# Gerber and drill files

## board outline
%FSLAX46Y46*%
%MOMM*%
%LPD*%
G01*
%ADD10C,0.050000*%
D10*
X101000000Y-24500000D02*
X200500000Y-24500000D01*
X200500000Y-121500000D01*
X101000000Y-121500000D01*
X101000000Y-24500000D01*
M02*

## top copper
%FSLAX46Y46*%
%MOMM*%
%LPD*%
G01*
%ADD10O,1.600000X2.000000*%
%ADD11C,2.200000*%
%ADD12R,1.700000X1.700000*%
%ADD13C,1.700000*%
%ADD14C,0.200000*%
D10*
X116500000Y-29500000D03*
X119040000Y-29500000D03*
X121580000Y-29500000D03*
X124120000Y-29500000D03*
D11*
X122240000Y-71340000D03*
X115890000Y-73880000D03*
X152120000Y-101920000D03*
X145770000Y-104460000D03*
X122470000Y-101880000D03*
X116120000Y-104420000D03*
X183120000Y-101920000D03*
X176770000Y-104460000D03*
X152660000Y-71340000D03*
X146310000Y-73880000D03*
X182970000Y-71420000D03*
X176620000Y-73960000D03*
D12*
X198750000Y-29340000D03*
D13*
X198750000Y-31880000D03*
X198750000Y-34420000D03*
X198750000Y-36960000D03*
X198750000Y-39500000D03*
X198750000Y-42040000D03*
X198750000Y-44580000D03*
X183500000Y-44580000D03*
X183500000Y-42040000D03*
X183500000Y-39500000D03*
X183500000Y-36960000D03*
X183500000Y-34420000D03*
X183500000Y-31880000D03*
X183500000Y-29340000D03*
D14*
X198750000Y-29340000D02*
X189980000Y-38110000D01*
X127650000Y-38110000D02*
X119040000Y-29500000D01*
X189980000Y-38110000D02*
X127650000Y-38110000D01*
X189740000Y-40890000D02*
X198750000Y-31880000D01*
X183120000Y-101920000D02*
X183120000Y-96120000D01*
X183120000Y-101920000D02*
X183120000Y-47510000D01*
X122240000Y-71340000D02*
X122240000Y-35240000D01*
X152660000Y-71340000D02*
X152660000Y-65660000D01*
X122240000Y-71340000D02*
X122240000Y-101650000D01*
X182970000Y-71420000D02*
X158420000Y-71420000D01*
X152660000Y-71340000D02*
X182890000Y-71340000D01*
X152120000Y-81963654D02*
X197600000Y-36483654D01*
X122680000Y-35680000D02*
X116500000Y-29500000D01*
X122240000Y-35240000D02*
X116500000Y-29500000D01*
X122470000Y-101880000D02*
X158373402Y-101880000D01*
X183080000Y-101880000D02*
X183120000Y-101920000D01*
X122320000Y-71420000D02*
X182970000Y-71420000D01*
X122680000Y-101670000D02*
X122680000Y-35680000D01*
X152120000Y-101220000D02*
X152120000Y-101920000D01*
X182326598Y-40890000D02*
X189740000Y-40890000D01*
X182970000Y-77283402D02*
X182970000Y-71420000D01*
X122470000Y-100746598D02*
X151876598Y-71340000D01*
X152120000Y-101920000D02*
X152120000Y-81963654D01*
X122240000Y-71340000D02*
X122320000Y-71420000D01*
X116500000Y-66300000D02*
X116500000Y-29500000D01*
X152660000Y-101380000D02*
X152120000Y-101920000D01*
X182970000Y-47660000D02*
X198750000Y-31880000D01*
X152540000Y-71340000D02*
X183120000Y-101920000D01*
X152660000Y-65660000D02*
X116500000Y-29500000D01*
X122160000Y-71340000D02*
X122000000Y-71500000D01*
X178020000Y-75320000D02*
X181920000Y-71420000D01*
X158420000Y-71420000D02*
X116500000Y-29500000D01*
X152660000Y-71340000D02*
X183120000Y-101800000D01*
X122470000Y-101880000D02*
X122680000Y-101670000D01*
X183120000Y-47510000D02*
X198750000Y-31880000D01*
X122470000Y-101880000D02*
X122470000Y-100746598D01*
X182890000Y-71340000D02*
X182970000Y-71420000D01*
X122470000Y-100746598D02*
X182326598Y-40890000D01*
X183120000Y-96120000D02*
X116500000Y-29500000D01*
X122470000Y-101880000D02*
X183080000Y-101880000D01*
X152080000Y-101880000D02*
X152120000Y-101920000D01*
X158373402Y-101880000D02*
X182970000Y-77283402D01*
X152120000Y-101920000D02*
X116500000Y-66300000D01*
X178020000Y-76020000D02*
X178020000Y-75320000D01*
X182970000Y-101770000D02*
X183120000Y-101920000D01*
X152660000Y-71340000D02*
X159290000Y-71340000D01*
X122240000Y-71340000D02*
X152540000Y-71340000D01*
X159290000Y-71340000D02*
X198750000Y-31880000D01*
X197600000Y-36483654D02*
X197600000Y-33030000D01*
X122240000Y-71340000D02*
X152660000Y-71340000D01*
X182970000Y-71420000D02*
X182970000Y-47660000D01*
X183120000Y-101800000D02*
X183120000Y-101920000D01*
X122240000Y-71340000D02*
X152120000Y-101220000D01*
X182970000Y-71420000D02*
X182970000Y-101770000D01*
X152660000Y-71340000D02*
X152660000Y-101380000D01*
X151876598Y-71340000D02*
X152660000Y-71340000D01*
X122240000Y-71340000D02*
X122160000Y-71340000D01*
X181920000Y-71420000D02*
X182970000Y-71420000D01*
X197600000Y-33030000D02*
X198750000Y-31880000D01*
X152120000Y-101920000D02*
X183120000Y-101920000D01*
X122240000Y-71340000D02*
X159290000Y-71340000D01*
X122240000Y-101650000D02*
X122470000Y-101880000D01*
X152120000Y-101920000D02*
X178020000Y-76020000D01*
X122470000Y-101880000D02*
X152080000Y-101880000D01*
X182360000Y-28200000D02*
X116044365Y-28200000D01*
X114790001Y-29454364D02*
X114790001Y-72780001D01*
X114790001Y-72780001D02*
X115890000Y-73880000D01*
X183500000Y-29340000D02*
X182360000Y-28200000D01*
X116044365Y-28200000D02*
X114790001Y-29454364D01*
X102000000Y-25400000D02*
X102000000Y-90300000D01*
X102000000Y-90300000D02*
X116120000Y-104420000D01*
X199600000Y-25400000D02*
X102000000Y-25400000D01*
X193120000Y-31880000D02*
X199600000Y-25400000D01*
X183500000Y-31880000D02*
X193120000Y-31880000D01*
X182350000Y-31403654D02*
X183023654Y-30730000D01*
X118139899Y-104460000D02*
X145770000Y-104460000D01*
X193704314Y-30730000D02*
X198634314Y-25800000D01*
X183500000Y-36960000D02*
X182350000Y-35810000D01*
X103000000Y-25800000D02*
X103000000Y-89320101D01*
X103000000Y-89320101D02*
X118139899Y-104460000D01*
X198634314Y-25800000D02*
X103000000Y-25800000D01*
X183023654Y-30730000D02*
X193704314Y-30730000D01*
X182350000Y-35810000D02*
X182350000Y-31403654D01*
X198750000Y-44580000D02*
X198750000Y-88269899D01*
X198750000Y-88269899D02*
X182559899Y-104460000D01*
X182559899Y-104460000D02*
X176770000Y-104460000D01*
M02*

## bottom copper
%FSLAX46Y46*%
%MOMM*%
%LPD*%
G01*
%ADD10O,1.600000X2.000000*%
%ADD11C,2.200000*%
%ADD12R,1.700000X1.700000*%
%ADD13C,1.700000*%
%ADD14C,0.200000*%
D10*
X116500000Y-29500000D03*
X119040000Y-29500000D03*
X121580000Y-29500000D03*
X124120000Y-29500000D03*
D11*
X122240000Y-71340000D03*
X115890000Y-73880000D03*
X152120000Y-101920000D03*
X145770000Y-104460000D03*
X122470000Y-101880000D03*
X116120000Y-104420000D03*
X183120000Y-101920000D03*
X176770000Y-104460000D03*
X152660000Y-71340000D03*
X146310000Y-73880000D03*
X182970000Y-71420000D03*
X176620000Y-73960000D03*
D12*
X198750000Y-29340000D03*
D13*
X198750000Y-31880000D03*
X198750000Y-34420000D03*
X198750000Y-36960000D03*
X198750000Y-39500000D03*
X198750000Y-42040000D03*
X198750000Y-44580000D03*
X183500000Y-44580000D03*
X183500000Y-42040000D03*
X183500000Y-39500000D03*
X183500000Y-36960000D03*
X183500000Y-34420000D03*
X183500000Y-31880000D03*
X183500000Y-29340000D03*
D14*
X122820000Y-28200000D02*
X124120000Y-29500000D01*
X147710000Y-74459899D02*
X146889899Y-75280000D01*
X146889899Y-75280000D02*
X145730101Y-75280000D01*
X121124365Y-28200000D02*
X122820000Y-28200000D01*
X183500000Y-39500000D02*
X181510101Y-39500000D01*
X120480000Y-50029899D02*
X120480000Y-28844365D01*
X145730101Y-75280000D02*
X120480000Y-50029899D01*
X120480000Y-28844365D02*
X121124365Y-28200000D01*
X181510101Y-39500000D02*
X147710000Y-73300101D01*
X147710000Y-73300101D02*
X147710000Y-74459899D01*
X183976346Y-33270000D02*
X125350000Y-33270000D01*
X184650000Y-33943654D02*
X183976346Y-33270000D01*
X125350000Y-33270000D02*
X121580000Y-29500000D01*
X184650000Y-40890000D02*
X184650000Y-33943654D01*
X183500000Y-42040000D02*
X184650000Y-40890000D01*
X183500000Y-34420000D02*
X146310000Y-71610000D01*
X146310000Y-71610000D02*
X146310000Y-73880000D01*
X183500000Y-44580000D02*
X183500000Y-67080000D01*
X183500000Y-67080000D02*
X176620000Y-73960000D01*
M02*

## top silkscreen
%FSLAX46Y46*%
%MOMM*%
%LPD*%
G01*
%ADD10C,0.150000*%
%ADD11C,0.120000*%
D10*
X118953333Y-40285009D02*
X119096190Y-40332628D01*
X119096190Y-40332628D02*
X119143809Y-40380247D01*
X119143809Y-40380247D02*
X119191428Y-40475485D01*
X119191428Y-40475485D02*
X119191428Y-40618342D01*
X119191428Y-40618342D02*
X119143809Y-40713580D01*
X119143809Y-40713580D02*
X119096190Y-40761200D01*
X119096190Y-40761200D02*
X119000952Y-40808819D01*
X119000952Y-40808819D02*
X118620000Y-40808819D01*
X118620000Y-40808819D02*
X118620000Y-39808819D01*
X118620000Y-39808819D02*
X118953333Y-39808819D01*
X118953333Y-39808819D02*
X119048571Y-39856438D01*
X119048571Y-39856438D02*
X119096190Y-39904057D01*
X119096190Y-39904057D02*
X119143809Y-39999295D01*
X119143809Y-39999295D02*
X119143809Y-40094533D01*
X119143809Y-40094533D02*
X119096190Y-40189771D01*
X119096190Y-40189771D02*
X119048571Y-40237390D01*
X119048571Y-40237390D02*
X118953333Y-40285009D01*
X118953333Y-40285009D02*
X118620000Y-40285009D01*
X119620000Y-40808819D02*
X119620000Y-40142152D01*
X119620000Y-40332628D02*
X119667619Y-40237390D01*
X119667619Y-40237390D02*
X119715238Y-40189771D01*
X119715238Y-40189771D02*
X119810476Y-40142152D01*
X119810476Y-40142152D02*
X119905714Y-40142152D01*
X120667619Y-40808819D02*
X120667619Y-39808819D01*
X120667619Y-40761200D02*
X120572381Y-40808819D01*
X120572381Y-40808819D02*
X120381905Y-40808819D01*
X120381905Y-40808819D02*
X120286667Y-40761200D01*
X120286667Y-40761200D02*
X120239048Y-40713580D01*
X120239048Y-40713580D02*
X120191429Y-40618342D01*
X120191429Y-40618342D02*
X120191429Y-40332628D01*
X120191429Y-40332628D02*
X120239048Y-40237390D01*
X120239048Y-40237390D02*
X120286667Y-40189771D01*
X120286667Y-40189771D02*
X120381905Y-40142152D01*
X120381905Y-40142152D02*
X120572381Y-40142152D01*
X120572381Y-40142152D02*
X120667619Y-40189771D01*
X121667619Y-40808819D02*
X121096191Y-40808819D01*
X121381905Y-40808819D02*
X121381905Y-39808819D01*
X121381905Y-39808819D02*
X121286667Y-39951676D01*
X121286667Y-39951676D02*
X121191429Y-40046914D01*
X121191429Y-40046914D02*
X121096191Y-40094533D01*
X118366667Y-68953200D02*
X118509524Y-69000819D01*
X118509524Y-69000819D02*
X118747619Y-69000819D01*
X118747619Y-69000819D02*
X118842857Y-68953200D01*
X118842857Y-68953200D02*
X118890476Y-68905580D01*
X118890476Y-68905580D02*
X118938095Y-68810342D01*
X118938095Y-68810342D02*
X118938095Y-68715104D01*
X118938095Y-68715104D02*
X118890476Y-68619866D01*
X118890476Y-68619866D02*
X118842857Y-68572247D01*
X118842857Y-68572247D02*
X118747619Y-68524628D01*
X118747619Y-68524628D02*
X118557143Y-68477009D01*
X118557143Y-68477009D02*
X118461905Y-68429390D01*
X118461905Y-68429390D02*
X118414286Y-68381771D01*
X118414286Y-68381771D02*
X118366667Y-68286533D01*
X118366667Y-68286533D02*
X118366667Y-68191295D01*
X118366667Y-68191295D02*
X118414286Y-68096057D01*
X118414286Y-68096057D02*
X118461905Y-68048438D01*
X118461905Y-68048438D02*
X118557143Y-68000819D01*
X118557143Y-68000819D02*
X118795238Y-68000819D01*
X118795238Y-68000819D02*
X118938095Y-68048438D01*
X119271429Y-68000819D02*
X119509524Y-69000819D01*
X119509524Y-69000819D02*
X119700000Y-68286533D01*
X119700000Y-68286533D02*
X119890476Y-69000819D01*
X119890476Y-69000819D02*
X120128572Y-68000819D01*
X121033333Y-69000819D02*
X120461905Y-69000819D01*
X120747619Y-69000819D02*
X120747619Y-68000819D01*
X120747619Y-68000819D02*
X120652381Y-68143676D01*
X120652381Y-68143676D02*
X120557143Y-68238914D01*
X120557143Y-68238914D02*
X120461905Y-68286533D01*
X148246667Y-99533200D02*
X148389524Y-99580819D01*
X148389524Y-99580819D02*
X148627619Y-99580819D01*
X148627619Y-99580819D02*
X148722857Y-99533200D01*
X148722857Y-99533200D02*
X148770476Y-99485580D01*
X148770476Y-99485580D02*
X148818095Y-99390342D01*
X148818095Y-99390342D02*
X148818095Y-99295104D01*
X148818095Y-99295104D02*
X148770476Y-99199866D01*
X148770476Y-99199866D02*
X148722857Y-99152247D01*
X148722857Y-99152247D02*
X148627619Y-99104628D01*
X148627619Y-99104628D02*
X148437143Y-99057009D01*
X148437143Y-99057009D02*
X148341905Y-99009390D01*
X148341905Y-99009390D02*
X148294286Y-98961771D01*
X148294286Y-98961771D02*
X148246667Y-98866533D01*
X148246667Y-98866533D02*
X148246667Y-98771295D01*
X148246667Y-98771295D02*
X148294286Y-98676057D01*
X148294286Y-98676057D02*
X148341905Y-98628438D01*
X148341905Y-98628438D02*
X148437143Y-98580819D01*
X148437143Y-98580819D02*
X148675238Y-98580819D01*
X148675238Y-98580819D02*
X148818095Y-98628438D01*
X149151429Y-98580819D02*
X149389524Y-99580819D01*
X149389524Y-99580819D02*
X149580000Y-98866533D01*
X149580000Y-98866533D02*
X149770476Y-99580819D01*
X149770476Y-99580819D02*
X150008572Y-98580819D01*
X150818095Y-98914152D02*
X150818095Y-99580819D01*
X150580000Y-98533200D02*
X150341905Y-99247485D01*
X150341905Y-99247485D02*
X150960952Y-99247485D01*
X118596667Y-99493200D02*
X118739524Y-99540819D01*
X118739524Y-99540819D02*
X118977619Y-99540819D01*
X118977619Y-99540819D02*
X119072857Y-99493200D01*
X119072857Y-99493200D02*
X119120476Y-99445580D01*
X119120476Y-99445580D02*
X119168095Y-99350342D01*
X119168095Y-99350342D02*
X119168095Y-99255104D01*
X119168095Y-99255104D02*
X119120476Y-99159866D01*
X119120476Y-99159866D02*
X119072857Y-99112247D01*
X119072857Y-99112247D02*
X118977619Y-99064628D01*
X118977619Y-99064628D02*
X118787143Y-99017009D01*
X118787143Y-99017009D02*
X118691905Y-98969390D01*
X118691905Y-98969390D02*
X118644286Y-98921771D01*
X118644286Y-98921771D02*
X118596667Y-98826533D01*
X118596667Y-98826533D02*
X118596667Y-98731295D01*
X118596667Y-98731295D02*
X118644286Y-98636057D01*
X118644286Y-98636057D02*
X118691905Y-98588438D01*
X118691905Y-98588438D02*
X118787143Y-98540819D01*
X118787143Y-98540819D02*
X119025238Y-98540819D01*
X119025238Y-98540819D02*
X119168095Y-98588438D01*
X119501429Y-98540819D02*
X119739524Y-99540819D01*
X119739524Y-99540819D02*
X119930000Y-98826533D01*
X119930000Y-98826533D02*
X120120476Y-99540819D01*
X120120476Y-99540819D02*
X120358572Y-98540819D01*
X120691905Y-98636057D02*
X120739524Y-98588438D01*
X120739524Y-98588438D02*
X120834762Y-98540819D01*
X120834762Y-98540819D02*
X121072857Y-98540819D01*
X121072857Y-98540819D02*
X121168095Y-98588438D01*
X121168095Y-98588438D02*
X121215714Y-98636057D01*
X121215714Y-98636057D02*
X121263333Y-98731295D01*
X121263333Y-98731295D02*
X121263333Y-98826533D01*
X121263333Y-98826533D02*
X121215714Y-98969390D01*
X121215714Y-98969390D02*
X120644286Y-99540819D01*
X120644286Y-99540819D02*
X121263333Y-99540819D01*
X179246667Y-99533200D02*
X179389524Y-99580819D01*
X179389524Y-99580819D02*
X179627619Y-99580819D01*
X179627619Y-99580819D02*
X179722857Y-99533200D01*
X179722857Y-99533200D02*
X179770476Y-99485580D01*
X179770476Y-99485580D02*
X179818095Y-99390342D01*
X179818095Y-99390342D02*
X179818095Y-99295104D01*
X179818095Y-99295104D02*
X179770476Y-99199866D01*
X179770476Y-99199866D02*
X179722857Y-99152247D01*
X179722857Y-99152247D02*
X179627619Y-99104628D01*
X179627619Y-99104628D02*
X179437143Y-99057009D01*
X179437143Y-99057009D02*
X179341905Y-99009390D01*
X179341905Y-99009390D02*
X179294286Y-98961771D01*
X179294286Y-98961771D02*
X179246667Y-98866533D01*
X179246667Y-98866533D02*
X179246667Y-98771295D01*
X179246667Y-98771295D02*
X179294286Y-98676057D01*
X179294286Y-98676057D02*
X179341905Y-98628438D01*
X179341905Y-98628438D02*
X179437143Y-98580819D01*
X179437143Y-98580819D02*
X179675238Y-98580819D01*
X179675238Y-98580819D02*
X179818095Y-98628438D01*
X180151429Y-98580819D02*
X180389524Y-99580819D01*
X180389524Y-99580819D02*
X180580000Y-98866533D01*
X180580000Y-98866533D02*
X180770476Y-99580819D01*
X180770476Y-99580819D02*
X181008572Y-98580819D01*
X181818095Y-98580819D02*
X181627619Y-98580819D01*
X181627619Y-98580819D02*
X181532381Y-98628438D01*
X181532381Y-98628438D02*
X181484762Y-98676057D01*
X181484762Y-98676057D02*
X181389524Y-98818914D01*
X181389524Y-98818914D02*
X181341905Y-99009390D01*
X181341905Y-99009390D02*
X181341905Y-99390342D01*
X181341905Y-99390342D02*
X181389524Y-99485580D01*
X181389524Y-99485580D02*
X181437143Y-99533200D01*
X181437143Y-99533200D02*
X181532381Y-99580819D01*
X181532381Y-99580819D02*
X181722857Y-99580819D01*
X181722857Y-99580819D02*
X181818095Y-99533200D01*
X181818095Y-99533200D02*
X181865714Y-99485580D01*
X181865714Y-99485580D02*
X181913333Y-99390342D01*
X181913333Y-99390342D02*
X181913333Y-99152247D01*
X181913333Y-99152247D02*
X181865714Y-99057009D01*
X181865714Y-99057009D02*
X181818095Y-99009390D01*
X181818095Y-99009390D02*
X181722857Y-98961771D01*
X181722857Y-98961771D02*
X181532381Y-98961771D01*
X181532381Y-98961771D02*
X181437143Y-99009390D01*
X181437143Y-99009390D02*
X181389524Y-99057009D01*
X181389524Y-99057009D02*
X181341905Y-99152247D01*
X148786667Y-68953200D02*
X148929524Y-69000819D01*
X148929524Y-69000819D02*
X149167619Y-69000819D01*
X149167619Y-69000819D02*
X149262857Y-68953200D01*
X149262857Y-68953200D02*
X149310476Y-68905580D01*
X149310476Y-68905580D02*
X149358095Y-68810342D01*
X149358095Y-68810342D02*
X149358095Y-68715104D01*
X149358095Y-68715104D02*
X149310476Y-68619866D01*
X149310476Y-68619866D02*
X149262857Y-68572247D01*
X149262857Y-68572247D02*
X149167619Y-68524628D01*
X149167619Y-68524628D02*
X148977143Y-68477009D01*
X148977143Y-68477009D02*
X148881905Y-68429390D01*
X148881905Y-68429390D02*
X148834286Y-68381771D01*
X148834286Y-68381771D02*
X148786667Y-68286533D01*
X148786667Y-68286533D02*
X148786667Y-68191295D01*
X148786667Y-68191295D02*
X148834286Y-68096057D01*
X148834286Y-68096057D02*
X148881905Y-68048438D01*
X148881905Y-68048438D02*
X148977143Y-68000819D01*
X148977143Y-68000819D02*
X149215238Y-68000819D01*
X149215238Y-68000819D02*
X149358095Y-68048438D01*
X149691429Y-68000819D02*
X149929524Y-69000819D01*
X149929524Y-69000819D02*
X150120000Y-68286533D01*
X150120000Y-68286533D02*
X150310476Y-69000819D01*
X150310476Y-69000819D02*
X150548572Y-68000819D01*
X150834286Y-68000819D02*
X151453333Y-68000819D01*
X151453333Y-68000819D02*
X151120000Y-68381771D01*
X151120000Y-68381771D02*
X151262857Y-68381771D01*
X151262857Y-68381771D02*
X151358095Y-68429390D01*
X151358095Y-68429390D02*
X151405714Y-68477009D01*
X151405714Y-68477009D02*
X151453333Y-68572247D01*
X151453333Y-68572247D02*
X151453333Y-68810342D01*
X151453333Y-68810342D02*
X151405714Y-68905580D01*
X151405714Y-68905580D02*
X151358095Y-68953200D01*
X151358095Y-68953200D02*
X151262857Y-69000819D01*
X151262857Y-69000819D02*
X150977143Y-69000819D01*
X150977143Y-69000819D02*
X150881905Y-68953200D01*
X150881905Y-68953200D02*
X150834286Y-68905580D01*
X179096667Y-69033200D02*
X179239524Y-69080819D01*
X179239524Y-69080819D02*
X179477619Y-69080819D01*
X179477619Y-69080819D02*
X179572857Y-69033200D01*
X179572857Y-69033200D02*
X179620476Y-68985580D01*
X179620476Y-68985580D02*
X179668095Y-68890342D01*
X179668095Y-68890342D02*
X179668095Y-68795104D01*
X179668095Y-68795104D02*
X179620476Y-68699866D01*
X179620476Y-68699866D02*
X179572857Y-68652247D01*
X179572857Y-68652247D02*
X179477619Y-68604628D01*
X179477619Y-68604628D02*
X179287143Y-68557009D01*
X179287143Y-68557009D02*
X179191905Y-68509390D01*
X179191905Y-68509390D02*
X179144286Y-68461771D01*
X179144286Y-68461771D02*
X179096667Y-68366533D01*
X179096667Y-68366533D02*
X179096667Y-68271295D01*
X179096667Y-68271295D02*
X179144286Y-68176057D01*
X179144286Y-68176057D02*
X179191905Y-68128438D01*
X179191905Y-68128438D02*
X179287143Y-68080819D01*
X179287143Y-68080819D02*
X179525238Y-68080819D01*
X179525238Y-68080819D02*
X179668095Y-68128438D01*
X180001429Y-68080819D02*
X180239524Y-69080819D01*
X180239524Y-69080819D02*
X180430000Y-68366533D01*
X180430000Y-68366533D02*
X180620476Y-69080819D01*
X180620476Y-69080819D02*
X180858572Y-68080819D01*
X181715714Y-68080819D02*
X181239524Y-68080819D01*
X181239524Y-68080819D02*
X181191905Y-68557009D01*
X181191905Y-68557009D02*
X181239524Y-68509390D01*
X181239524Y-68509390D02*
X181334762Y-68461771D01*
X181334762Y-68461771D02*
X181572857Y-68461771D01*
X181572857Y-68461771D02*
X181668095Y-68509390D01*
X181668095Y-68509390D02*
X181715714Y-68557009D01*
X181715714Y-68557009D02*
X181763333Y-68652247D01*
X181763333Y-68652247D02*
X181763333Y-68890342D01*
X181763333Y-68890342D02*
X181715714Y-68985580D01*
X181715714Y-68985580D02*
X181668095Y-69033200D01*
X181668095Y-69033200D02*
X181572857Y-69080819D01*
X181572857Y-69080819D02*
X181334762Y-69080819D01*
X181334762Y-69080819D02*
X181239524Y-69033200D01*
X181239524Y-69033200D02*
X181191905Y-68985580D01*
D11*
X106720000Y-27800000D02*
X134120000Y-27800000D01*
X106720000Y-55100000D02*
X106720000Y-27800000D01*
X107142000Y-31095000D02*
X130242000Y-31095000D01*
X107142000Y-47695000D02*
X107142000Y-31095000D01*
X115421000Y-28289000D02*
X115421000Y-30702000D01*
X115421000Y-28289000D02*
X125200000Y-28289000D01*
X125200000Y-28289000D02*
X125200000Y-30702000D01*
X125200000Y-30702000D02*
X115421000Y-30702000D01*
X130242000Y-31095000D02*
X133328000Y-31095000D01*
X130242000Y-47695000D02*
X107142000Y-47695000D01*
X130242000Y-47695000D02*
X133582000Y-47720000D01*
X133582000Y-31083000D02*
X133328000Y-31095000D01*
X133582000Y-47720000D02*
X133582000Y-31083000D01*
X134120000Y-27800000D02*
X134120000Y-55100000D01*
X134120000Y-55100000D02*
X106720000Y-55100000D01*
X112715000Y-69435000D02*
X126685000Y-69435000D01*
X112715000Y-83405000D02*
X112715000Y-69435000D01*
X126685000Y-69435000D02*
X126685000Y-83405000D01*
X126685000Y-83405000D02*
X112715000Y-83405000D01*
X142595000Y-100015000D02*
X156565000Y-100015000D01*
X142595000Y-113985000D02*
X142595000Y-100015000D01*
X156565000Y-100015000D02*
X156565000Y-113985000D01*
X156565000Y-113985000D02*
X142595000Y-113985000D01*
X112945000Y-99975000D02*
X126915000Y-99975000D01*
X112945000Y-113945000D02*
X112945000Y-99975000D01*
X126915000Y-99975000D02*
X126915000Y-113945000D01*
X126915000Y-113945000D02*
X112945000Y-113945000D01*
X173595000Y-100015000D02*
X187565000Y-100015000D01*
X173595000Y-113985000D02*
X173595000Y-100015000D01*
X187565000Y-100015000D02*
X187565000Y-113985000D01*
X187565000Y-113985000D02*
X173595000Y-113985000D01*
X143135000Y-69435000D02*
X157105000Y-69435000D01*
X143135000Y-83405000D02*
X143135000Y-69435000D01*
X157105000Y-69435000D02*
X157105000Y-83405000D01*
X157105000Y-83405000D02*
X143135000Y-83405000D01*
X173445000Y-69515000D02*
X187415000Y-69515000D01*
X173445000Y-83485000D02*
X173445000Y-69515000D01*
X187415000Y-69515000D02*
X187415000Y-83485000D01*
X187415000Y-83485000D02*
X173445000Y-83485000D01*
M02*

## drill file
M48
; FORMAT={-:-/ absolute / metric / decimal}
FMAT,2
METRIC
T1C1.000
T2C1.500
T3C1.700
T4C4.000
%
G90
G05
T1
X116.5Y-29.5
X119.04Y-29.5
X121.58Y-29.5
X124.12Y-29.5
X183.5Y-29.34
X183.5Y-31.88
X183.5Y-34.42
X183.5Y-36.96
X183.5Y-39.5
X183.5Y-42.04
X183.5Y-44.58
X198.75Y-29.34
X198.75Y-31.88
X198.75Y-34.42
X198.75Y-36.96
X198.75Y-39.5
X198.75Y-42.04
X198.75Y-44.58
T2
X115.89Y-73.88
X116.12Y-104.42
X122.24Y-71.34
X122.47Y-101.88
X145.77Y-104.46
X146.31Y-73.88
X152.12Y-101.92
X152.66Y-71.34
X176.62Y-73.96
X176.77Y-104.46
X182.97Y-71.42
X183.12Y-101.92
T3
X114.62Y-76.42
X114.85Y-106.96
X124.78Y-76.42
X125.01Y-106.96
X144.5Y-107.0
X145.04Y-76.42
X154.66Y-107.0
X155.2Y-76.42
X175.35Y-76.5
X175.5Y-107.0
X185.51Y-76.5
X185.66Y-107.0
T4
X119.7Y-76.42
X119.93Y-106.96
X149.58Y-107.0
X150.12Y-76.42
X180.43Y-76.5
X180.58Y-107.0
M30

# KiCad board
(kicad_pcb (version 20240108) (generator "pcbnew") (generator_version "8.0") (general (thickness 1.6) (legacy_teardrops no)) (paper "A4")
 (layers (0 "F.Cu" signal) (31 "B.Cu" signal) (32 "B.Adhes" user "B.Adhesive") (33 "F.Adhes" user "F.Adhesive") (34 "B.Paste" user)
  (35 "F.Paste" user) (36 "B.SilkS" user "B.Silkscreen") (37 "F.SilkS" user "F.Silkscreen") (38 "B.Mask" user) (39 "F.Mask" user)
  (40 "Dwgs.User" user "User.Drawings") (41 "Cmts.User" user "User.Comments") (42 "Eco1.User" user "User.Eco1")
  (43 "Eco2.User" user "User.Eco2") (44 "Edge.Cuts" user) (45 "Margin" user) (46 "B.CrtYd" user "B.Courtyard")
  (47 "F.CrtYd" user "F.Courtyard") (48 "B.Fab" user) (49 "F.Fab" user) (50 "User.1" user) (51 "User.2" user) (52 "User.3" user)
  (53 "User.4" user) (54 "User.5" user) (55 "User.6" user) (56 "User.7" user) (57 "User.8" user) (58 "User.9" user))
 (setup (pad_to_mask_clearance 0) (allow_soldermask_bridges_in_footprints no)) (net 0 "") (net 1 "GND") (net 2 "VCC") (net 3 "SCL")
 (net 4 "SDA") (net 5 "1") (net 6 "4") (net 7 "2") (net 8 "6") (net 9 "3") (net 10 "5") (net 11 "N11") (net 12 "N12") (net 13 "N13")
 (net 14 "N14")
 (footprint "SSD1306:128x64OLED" (layer "F.Cu") (at 120.12 40.1)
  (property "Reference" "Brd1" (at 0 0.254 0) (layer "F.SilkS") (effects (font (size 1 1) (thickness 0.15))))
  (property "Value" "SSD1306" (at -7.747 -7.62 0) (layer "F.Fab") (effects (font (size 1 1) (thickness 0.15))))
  (fp_line (start -13.4 -12.3) (end 14 -12.3) (stroke (width 0.12) (type solid)) (layer "F.SilkS"))
  (fp_line (start -13.4 15) (end -13.4 -12.3) (stroke (width 0.12) (type solid)) (layer "F.SilkS"))
  (fp_line (start -12.978 -9.005) (end 10.122 -9.005) (stroke (width 0.12) (type solid)) (layer "F.SilkS"))
  (fp_line (start -12.978 7.595) (end -12.978 -9.005) (stroke (width 0.12) (type solid)) (layer "F.SilkS"))
  (fp_line (start -4.699 -11.811) (end -4.699 -9.398) (stroke (width 0.12) (type solid)) (layer "F.SilkS"))
  (fp_line (start -4.699 -11.811) (end 5.08 -11.811) (stroke (width 0.12) (type solid)) (layer "F.SilkS"))
  (fp_line (start 5.08 -11.811) (end 5.08 -9.398) (stroke (width 0.12) (type solid)) (layer "F.SilkS"))
  (fp_line (start 5.08 -9.398) (end -4.699 -9.398) (stroke (width 0.12) (type solid)) (layer "F.SilkS"))
  (fp_line (start 10.122 -9.005) (end 13.208 -9.005) (stroke (width 0.12) (type solid)) (layer "F.SilkS"))
  (fp_line (start 10.122 7.595) (end -12.978 7.595) (stroke (width 0.12) (type solid)) (layer "F.SilkS"))
  (fp_line (start 10.122 7.595) (end 13.462 7.62) (stroke (width 0.12) (type solid)) (layer "F.SilkS"))
  (fp_line (start 13.462 -9.017) (end 13.208 -9.005) (stroke (width 0.12) (type solid)) (layer "F.SilkS"))
  (fp_line (start 13.462 7.62) (end 13.462 -9.017) (stroke (width 0.12) (type solid)) (layer "F.SilkS"))
  (fp_line (start 14 -12.3) (end 14 15) (stroke (width 0.12) (type solid)) (layer "F.SilkS"))
  (fp_line (start 14 15) (end -13.4 15) (stroke (width 0.12) (type solid)) (layer "F.SilkS"))
  (pad "1" thru_hole oval (at -3.62 -10.6 90) (size 2 1.6) (drill 1) (layers "*.Cu" "*.Mask") (remove_unused_layers no) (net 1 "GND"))
  (pad "2" thru_hole oval (at -1.08 -10.6 90) (size 2 1.6) (drill 1) (layers "*.Cu" "*.Mask") (remove_unused_layers no) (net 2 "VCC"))
  (pad "3" thru_hole oval (at 1.46 -10.6 90) (size 2 1.6) (drill 1) (layers "*.Cu" "*.Mask") (remove_unused_layers no) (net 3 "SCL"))
  (pad "4" thru_hole oval (at 4 -10.6 90) (size 2 1.6) (drill 1) (layers "*.Cu" "*.Mask") (remove_unused_layers no) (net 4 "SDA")))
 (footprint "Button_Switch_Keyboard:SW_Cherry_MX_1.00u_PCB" (layer "F.Cu") (at 122.24 71.34)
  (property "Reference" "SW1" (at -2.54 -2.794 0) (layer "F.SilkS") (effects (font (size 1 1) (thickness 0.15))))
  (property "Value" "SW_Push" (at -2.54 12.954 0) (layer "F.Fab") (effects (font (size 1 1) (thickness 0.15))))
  (fp_line (start -9.525 -1.905) (end 4.445 -1.905) (stroke (width 0.12) (type solid)) (layer "F.SilkS"))
  (fp_line (start -9.525 12.065) (end -9.525 -1.905) (stroke (width 0.12) (type solid)) (layer "F.SilkS"))
  (fp_line (start 4.445 -1.905) (end 4.445 12.065) (stroke (width 0.12) (type solid)) (layer "F.SilkS"))
  (fp_line (start 4.445 12.065) (end -9.525 12.065) (stroke (width 0.12) (type solid)) (layer "F.SilkS"))
  (pad "" np_thru_hole circle (at -7.62 5.08) (size 1.7 1.7) (drill 1.7) (layers "*.Cu" "*.Mask"))
  (pad "" np_thru_hole circle (at -2.54 5.08) (size 4 4) (drill 4) (layers "*.Cu" "*.Mask"))
  (pad "" np_thru_hole circle (at 2.54 5.08) (size 1.7 1.7) (drill 1.7) (layers "*.Cu" "*.Mask"))
  (pad "1" thru_hole circle (at 0 0) (size 2.2 2.2) (drill 1.5) (layers "*.Cu" "*.Mask") (remove_unused_layers no) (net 1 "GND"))
  (pad "2" thru_hole circle (at -6.35 2.54) (size 2.2 2.2) (drill 1.5) (layers "*.Cu" "*.Mask") (remove_unused_layers no) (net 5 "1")))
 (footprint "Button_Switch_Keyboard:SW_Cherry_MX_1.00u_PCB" (layer "F.Cu") (at 152.12 101.92)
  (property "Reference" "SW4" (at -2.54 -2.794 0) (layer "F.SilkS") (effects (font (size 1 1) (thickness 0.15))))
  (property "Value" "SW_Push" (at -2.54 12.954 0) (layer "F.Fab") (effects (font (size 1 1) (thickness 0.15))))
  (fp_line (start -9.525 -1.905) (end 4.445 -1.905) (stroke (width 0.12) (type solid)) (layer "F.SilkS"))
  (fp_line (start -9.525 12.065) (end -9.525 -1.905) (stroke (width 0.12) (type solid)) (layer "F.SilkS"))
  (fp_line (start 4.445 -1.905) (end 4.445 12.065) (stroke (width 0.12) (type solid)) (layer "F.SilkS"))
  (fp_line (start 4.445 12.065) (end -9.525 12.065) (stroke (width 0.12) (type solid)) (layer "F.SilkS"))
  (pad "" np_thru_hole circle (at -7.62 5.08) (size 1.7 1.7) (drill 1.7) (layers "*.Cu" "*.Mask"))
  (pad "" np_thru_hole circle (at -2.54 5.08) (size 4 4) (drill 4) (layers "*.Cu" "*.Mask"))
  (pad "" np_thru_hole circle (at 2.54 5.08) (size 1.7 1.7) (drill 1.7) (layers "*.Cu" "*.Mask"))
  (pad "1" thru_hole circle (at 0 0) (size 2.2 2.2) (drill 1.5) (layers "*.Cu" "*.Mask") (remove_unused_layers no) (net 1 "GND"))
  (pad "2" thru_hole circle (at -6.35 2.54) (size 2.2 2.2) (drill 1.5) (layers "*.Cu" "*.Mask") (remove_unused_layers no) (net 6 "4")))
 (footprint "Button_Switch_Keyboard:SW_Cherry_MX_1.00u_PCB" (layer "F.Cu") (at 122.47 101.88)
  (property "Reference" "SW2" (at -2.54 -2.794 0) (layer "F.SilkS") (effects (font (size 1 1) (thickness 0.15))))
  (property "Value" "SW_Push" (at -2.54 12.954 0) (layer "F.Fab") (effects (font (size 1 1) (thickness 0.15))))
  (fp_line (start -9.525 -1.905) (end 4.445 -1.905) (stroke (width 0.12) (type solid)) (layer "F.SilkS"))
  (fp_line (start -9.525 12.065) (end -9.525 -1.905) (stroke (width 0.12) (type solid)) (layer "F.SilkS"))
  (fp_line (start 4.445 -1.905) (end 4.445 12.065) (stroke (width 0.12) (type solid)) (layer "F.SilkS"))
  (fp_line (start 4.445 12.065) (end -9.525 12.065) (stroke (width 0.12) (type solid)) (layer "F.SilkS"))
  (pad "" np_thru_hole circle (at -7.62 5.08) (size 1.7 1.7) (drill 1.7) (layers "*.Cu" "*.Mask"))
  (pad "" np_thru_hole circle (at -2.54 5.08) (size 4 4) (drill 4) (layers "*.Cu" "*.Mask"))
  (pad "" np_thru_hole circle (at 2.54 5.08) (size 1.7 1.7) (drill 1.7) (layers "*.Cu" "*.Mask"))
  (pad "1" thru_hole circle (at 0 0) (size 2.2 2.2) (drill 1.5) (layers "*.Cu" "*.Mask") (remove_unused_layers no) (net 1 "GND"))
  (pad "2" thru_hole circle (at -6.35 2.54) (size 2.2 2.2) (drill 1.5) (layers "*.Cu" "*.Mask") (remove_unused_layers no) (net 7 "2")))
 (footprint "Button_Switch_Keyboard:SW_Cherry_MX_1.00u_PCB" (layer "F.Cu") (at 183.12 101.92)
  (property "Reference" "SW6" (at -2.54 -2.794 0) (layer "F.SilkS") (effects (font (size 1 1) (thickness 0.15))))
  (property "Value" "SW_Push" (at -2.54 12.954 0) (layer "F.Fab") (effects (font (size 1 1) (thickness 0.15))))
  (fp_line (start -9.525 -1.905) (end 4.445 -1.905) (stroke (width 0.12) (type solid)) (layer "F.SilkS"))
  (fp_line (start -9.525 12.065) (end -9.525 -1.905) (stroke (width 0.12) (type solid)) (layer "F.SilkS"))
  (fp_line (start 4.445 -1.905) (end 4.445 12.065) (stroke (width 0.12) (type solid)) (layer "F.SilkS"))
  (fp_line (start 4.445 12.065) (end -9.525 12.065) (stroke (width 0.12) (type solid)) (layer "F.SilkS"))
  (pad "" np_thru_hole circle (at -7.62 5.08) (size 1.7 1.7) (drill 1.7) (layers "*.Cu" "*.Mask"))
  (pad "" np_thru_hole circle (at -2.54 5.08) (size 4 4) (drill 4) (layers "*.Cu" "*.Mask"))
  (pad "" np_thru_hole circle (at 2.54 5.08) (size 1.7 1.7) (drill 1.7) (layers "*.Cu" "*.Mask"))
  (pad "1" thru_hole circle (at 0 0) (size 2.2 2.2) (drill 1.5) (layers "*.Cu" "*.Mask") (remove_unused_layers no) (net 1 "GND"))
  (pad "2" thru_hole circle (at -6.35 2.54) (size 2.2 2.2) (drill 1.5) (layers "*.Cu" "*.Mask") (remove_unused_layers no) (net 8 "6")))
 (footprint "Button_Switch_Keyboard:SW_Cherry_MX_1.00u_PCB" (layer "F.Cu") (at 152.66 71.34)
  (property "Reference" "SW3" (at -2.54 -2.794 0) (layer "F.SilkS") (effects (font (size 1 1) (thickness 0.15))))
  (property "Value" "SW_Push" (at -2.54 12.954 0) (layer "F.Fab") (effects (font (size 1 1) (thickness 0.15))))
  (fp_line (start -9.525 -1.905) (end 4.445 -1.905) (stroke (width 0.12) (type solid)) (layer "F.SilkS"))
  (fp_line (start -9.525 12.065) (end -9.525 -1.905) (stroke (width 0.12) (type solid)) (layer "F.SilkS"))
  (fp_line (start 4.445 -1.905) (end 4.445 12.065) (stroke (width 0.12) (type solid)) (layer "F.SilkS"))
  (fp_line (start 4.445 12.065) (end -9.525 12.065) (stroke (width 0.12) (type solid)) (layer "F.SilkS"))
  (pad "" np_thru_hole circle (at -7.62 5.08) (size 1.7 1.7) (drill 1.7) (layers "*.Cu" "*.Mask"))
  (pad "" np_thru_hole circle (at -2.54 5.08) (size 4 4) (drill 4) (layers "*.Cu" "*.Mask"))
  (pad "" np_thru_hole circle (at 2.54 5.08) (size 1.7 1.7) (drill 1.7) (layers "*.Cu" "*.Mask"))
  (pad "1" thru_hole circle (at 0 0) (size 2.2 2.2) (drill 1.5) (layers "*.Cu" "*.Mask") (remove_unused_layers no) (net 1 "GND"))
  (pad "2" thru_hole circle (at -6.35 2.54) (size 2.2 2.2) (drill 1.5) (layers "*.Cu" "*.Mask") (remove_unused_layers no) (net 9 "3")))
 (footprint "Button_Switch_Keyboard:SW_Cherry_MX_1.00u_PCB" (layer "F.Cu") (at 182.97 71.42)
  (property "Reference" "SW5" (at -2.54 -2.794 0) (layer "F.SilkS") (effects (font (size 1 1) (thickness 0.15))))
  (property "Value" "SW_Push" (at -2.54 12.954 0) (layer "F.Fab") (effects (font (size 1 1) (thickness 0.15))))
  (fp_line (start -9.525 -1.905) (end 4.445 -1.905) (stroke (width 0.12) (type solid)) (layer "F.SilkS"))
  (fp_line (start -9.525 12.065) (end -9.525 -1.905) (stroke (width 0.12) (type solid)) (layer "F.SilkS"))
  (fp_line (start 4.445 -1.905) (end 4.445 12.065) (stroke (width 0.12) (type solid)) (layer "F.SilkS"))
  (fp_line (start 4.445 12.065) (end -9.525 12.065) (stroke (width 0.12) (type solid)) (layer "F.SilkS"))
  (pad "" np_thru_hole circle (at -7.62 5.08) (size 1.7 1.7) (drill 1.7) (layers "*.Cu" "*.Mask"))
  (pad "" np_thru_hole circle (at -2.54 5.08) (size 4 4) (drill 4) (layers "*.Cu" "*.Mask"))
  (pad "" np_thru_hole circle (at 2.54 5.08) (size 1.7 1.7) (drill 1.7) (layers "*.Cu" "*.Mask"))
  (pad "1" thru_hole circle (at 0 0) (size 2.2 2.2) (drill 1.5) (layers "*.Cu" "*.Mask") (remove_unused_layers no) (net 1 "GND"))
  (pad "2" thru_hole circle (at -6.35 2.54) (size 2.2 2.2) (drill 1.5) (layers "*.Cu" "*.Mask") (remove_unused_layers no) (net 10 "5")))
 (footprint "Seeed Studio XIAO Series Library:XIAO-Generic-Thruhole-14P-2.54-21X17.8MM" (layer "B.Cu") (at 191.125 36.96 180)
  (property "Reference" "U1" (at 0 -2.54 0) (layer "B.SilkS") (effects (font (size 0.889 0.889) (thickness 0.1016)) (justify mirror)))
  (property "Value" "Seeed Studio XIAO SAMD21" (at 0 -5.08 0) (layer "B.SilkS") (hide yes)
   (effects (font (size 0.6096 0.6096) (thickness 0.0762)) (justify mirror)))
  (pad "1" thru_hole rect (at -7.625 7.62 180) (size 1.7 1.7) (drill 1) (layers "*.Cu" "*.Mask") (remove_unused_layers no) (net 2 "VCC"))
  (pad "2" thru_hole circle (at -7.625 5.08 180) (size 1.7 1.7) (drill 1) (layers "*.Cu" "*.Mask") (remove_unused_layers no) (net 1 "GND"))
  (pad "3" thru_hole circle (at -7.625 2.54 180) (size 1.7 1.7) (drill 1) (layers "*.Cu" "*.Mask") (remove_unused_layers no) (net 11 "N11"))
  (pad "4" thru_hole circle (at -7.625 0 180) (size 1.7 1.7) (drill 1) (layers "*.Cu" "*.Mask") (remove_unused_layers no) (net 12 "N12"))
  (pad "5" thru_hole circle (at -7.625 -2.54 180) (size 1.7 1.7) (drill 1) (layers "*.Cu" "*.Mask") (remove_unused_layers no) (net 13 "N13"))
  (pad "6" thru_hole circle (at -7.625 -5.08) (size 1.7 1.7) (drill 1) (layers "*.Cu" "*.Mask") (remove_unused_layers no) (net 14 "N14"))
  (pad "7" thru_hole circle (at -7.625 -7.62 180) (size 1.7 1.7) (drill 1) (layers "*.Cu" "*.Mask") (remove_unused_layers no) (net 8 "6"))
  (pad "8" thru_hole circle (at 7.625 -7.62 180) (size 1.7 1.7) (drill 1) (layers "*.Cu" "*.Mask") (remove_unused_layers no) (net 10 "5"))
  (pad "9" thru_hole circle (at 7.625 -5.08 180) (size 1.7 1.7) (drill 1) (layers "*.Cu" "*.Mask") (remove_unused_layers no) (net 3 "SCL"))
  (pad "10" thru_hole circle (at 7.625 -2.54 180) (size 1.7 1.7) (drill 1) (layers "*.Cu" "*.Mask") (remove_unused_layers no) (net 4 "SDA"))
  (pad "11" thru_hole circle (at 7.625 0 180) (size 1.7 1.7) (drill 1) (layers "*.Cu" "*.Mask") (remove_unused_layers no) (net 6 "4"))
  (pad "12" thru_hole circle (at 7.625 2.54 180) (size 1.7 1.7) (drill 1) (layers "*.Cu" "*.Mask") (remove_unused_layers no) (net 9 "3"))
  (pad "13" thru_hole circle (at 7.625 5.08 180) (size 1.7 1.7) (drill 1) (layers "*.Cu" "*.Mask") (remove_unused_layers no) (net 7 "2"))
  (pad "14" thru_hole circle (at 7.625 7.62 180) (size 1.7 1.7) (drill 1) (layers "*.Cu" "*.Mask") (remove_unused_layers no) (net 5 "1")))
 (gr_rect (start 101 24.5) (end 200.5 121.5) (stroke (width 0.05) (type default)) (fill none) (layer "Edge.Cuts"))
 (segment (start 198.75 29.34) (end 189.98 38.11) (width 0.2) (layer "F.Cu") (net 2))
 (segment (start 127.65 38.11) (end 119.04 29.5) (width 0.2) (layer "F.Cu") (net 2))
 (segment (start 189.98 38.11) (end 127.65 38.11) (width 0.2) (layer "F.Cu") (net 2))
 (segment (start 189.74 40.89) (end 198.75 31.88) (width 0.2) (layer "F.Cu") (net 1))
 (segment (start 183.12 101.92) (end 183.12 96.12) (width 0.2) (layer "F.Cu") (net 1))
 (segment (start 183.12 101.92) (end 183.12 47.51) (width 0.2) (layer "F.Cu") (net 1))
 (segment (start 122.24 71.34) (end 122.24 35.24) (width 0.2) (layer "F.Cu") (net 1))
 (segment (start 152.66 71.34) (end 152.66 65.66) (width 0.2) (layer "F.Cu") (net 1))
 (segment (start 122.24 71.34) (end 122.24 101.65) (width 0.2) (layer "F.Cu") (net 1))
 (segment (start 182.97 71.42) (end 158.42 71.42) (width 0.2) (layer "F.Cu") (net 1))
 (segment (start 152.66 71.34) (end 182.89 71.34) (width 0.2) (layer "F.Cu") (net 1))
 (segment (start 152.12 81.963654) (end 197.6 36.483654) (width 0.2) (layer "F.Cu") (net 1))
 (segment (start 122.68 35.68) (end 116.5 29.5) (width 0.2) (layer "F.Cu") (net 1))
 (segment (start 122.24 35.24) (end 116.5 29.5) (width 0.2) (layer "F.Cu") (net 1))
 (segment (start 122.47 101.88) (end 158.373402 101.88) (width 0.2) (layer "F.Cu") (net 1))
 (segment (start 183.08 101.88) (end 183.12 101.92) (width 0.2) (layer "F.Cu") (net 1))
 (segment (start 122.32 71.42) (end 182.97 71.42) (width 0.2) (layer "F.Cu") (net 1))
 (segment (start 122.68 101.67) (end 122.68 35.68) (width 0.2) (layer "F.Cu") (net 1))
 (segment (start 152.12 101.22) (end 152.12 101.92) (width 0.2) (layer "F.Cu") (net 1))
 (segment (start 182.326598 40.89) (end 189.74 40.89) (width 0.2) (layer "F.Cu") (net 1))
 (segment (start 182.97 77.283402) (end 182.97 71.42) (width 0.2) (layer "F.Cu") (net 1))
 (segment (start 122.47 100.746598) (end 151.876598 71.34) (width 0.2) (layer "F.Cu") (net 1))
 (segment (start 152.12 101.92) (end 152.12 81.963654) (width 0.2) (layer "F.Cu") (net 1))
 (segment (start 122.24 71.34) (end 122.32 71.42) (width 0.2) (layer "F.Cu") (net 1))
 (segment (start 116.5 66.3) (end 116.5 29.5) (width 0.2) (layer "F.Cu") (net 1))
 (segment (start 152.66 101.38) (end 152.12 101.92) (width 0.2) (layer "F.Cu") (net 1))
 (segment (start 182.97 47.66) (end 198.75 31.88) (width 0.2) (layer "F.Cu") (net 1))
 (segment (start 152.54 71.34) (end 183.12 101.92) (width 0.2) (layer "F.Cu") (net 1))
 (segment (start 152.66 65.66) (end 116.5 29.5) (width 0.2) (layer "F.Cu") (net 1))
 (segment (start 122.16 71.34) (end 122 71.5) (width 0.2) (layer "F.Cu") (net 1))
 (segment (start 178.02 75.32) (end 181.92 71.42) (width 0.2) (layer "F.Cu") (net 1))
 (segment (start 158.42 71.42) (end 116.5 29.5) (width 0.2) (layer "F.Cu") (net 1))
 (segment (start 152.66 71.34) (end 183.12 101.8) (width 0.2) (layer "F.Cu") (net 1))
 (segment (start 122.47 101.88) (end 122.68 101.67) (width 0.2) (layer "F.Cu") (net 1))
 (segment (start 183.12 47.51) (end 198.75 31.88) (width 0.2) (layer "F.Cu") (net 1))
 (segment (start 122.47 101.88) (end 122.47 100.746598) (width 0.2) (layer "F.Cu") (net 1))
 (segment (start 182.89 71.34) (end 182.97 71.42) (width 0.2) (layer "F.Cu") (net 1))
 (segment (start 122.47 100.746598) (end 182.326598 40.89) (width 0.2) (layer "F.Cu") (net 1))
 (segment (start 183.12 96.12) (end 116.5 29.5) (width 0.2) (layer "F.Cu") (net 1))
 (segment (start 122.47 101.88) (end 183.08 101.88) (width 0.2) (layer "F.Cu") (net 1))
 (segment (start 152.08 101.88) (end 152.12 101.92) (width 0.2) (layer "F.Cu") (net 1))
 (segment (start 158.373402 101.88) (end 182.97 77.283402) (width 0.2) (layer "F.Cu") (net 1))
 (segment (start 152.12 101.92) (end 116.5 66.3) (width 0.2) (layer "F.Cu") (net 1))
 (segment (start 178.02 76.02) (end 178.02 75.32) (width 0.2) (layer "F.Cu") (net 1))
 (segment (start 182.97 101.77) (end 183.12 101.92) (width 0.2) (layer "F.Cu") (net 1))
 (segment (start 152.66 71.34) (end 159.29 71.34) (width 0.2) (layer "F.Cu") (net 1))
 (segment (start 122.24 71.34) (end 152.54 71.34) (width 0.2) (layer "F.Cu") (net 1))
 (segment (start 159.29 71.34) (end 198.75 31.88) (width 0.2) (layer "F.Cu") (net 1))
 (segment (start 197.6 36.483654) (end 197.6 33.03) (width 0.2) (layer "F.Cu") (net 1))
 (segment (start 122.24 71.34) (end 152.66 71.34) (width 0.2) (layer "F.Cu") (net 1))
 (segment (start 182.97 71.42) (end 182.97 47.66) (width 0.2) (layer "F.Cu") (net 1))
 (segment (start 183.12 101.8) (end 183.12 101.92) (width 0.2) (layer "F.Cu") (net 1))
 (segment (start 122.24 71.34) (end 152.12 101.22) (width 0.2) (layer "F.Cu") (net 1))
 (segment (start 182.97 71.42) (end 182.97 101.77) (width 0.2) (layer "F.Cu") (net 1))
 (segment (start 152.66 71.34) (end 152.66 101.38) (width 0.2) (layer "F.Cu") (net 1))
 (segment (start 151.876598 71.34) (end 152.66 71.34) (width 0.2) (layer "F.Cu") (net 1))
 (segment (start 122.24 71.34) (end 122.16 71.34) (width 0.2) (layer "F.Cu") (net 1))
 (segment (start 181.92 71.42) (end 182.97 71.42) (width 0.2) (layer "F.Cu") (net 1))
 (segment (start 197.6 33.03) (end 198.75 31.88) (width 0.2) (layer "F.Cu") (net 1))
 (segment (start 152.12 101.92) (end 183.12 101.92) (width 0.2) (layer "F.Cu") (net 1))
 (segment (start 122.24 71.34) (end 159.29 71.34) (width 0.2) (layer "F.Cu") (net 1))
 (segment (start 122.24 101.65) (end 122.47 101.88) (width 0.2) (layer "F.Cu") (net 1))
 (segment (start 152.12 101.92) (end 178.02 76.02) (width 0.2) (layer "F.Cu") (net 1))
 (segment (start 122.47 101.88) (end 152.08 101.88) (width 0.2) (layer "F.Cu") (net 1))
 (segment (start 122.82 28.2) (end 124.12 29.5) (width 0.2) (layer "B.Cu") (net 4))
 (segment (start 147.71 74.459899) (end 146.889899 75.28) (width 0.2) (layer "B.Cu") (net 4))
 (segment (start 146.889899 75.28) (end 145.730101 75.28) (width 0.2) (layer "B.Cu") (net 4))
 (segment (start 121.124365 28.2) (end 122.82 28.2) (width 0.2) (layer "B.Cu") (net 4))
 (segment (start 183.5 39.5) (end 181.510101 39.5) (width 0.2) (layer "B.Cu") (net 4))
 (segment (start 120.48 50.029899) (end 120.48 28.844365) (width 0.2) (layer "B.Cu") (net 4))
 (segment (start 145.730101 75.28) (end 120.48 50.029899) (width 0.2) (layer "B.Cu") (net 4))
 (segment (start 120.48 28.844365) (end 121.124365 28.2) (width 0.2) (layer "B.Cu") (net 4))
 (segment (start 181.510101 39.5) (end 147.71 73.300101) (width 0.2) (layer "B.Cu") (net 4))
 (segment (start 147.71 73.300101) (end 147.71 74.459899) (width 0.2) (layer "B.Cu") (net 4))
 (segment (start 183.976346 33.27) (end 125.35 33.27) (width 0.2) (layer "B.Cu") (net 3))
 (segment (start 184.65 33.943654) (end 183.976346 33.27) (width 0.2) (layer "B.Cu") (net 3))
 (segment (start 125.35 33.27) (end 121.58 29.5) (width 0.2) (layer "B.Cu") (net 3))
 (segment (start 184.65 40.89) (end 184.65 33.943654) (width 0.2) (layer "B.Cu") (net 3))
 (segment (start 183.5 42.04) (end 184.65 40.89) (width 0.2) (layer "B.Cu") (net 3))
 (segment (start 182.36 28.2) (end 116.044365 28.2) (width 0.2) (layer "F.Cu") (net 5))
 (segment (start 114.790001 29.454364) (end 114.790001 72.780001) (width 0.2) (layer "F.Cu") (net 5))
 (segment (start 114.790001 72.780001) (end 115.89 73.88) (width 0.2) (layer "F.Cu") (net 5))
 (segment (start 183.5 29.34) (end 182.36 28.2) (width 0.2) (layer "F.Cu") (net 5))
 (segment (start 116.044365 28.2) (end 114.790001 29.454364) (width 0.2) (layer "F.Cu") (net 5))
 (segment (start 102 25.4) (end 102 90.3) (width 0.2) (layer "F.Cu") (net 7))
 (segment (start 102 90.3) (end 116.12 104.42) (width 0.2) (layer "F.Cu") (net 7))
 (segment (start 199.6 25.4) (end 102 25.4) (width 0.2) (layer "F.Cu") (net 7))
 (segment (start 193.12 31.88) (end 199.6 25.4) (width 0.2) (layer "F.Cu") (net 7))
 (segment (start 183.5 31.88) (end 193.12 31.88) (width 0.2) (layer "F.Cu") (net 7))
 (segment (start 183.5 34.42) (end 146.31 71.61) (width 0.2) (layer "B.Cu") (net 9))
 (segment (start 146.31 71.61) (end 146.31 73.88) (width 0.2) (layer "B.Cu") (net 9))
 (segment (start 182.35 31.403654) (end 183.023654 30.73) (width 0.2) (layer "F.Cu") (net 6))
 (segment (start 118.139899 104.46) (end 145.77 104.46) (width 0.2) (layer "F.Cu") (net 6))
 (segment (start 193.704314 30.73) (end 198.634314 25.8) (width 0.2) (layer "F.Cu") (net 6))
 (segment (start 183.5 36.96) (end 182.35 35.81) (width 0.2) (layer "F.Cu") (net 6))
 (segment (start 103 25.8) (end 103 89.320101) (width 0.2) (layer "F.Cu") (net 6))
 (segment (start 103 89.320101) (end 118.139899 104.46) (width 0.2) (layer "F.Cu") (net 6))
 (segment (start 198.634314 25.8) (end 103 25.8) (width 0.2) (layer "F.Cu") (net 6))
 (segment (start 183.023654 30.73) (end 193.704314 30.73) (width 0.2) (layer "F.Cu") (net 6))
 (segment (start 182.35 35.81) (end 182.35 31.403654) (width 0.2) (layer "F.Cu") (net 6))
 (segment (start 183.5 44.58) (end 183.5 67.08) (width 0.2) (layer "B.Cu") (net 10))
 (segment (start 183.5 67.08) (end 176.62 73.96) (width 0.2) (layer "B.Cu") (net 10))
 (segment (start 198.75 44.58) (end 198.75 88.269899) (width 0.2) (layer "F.Cu") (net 8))
 (segment (start 198.75 88.269899) (end 182.559899 104.46) (width 0.2) (layer "F.Cu") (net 8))
 (segment (start 182.559899 104.46) (end 176.77 104.46) (width 0.2) (layer "F.Cu") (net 8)))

